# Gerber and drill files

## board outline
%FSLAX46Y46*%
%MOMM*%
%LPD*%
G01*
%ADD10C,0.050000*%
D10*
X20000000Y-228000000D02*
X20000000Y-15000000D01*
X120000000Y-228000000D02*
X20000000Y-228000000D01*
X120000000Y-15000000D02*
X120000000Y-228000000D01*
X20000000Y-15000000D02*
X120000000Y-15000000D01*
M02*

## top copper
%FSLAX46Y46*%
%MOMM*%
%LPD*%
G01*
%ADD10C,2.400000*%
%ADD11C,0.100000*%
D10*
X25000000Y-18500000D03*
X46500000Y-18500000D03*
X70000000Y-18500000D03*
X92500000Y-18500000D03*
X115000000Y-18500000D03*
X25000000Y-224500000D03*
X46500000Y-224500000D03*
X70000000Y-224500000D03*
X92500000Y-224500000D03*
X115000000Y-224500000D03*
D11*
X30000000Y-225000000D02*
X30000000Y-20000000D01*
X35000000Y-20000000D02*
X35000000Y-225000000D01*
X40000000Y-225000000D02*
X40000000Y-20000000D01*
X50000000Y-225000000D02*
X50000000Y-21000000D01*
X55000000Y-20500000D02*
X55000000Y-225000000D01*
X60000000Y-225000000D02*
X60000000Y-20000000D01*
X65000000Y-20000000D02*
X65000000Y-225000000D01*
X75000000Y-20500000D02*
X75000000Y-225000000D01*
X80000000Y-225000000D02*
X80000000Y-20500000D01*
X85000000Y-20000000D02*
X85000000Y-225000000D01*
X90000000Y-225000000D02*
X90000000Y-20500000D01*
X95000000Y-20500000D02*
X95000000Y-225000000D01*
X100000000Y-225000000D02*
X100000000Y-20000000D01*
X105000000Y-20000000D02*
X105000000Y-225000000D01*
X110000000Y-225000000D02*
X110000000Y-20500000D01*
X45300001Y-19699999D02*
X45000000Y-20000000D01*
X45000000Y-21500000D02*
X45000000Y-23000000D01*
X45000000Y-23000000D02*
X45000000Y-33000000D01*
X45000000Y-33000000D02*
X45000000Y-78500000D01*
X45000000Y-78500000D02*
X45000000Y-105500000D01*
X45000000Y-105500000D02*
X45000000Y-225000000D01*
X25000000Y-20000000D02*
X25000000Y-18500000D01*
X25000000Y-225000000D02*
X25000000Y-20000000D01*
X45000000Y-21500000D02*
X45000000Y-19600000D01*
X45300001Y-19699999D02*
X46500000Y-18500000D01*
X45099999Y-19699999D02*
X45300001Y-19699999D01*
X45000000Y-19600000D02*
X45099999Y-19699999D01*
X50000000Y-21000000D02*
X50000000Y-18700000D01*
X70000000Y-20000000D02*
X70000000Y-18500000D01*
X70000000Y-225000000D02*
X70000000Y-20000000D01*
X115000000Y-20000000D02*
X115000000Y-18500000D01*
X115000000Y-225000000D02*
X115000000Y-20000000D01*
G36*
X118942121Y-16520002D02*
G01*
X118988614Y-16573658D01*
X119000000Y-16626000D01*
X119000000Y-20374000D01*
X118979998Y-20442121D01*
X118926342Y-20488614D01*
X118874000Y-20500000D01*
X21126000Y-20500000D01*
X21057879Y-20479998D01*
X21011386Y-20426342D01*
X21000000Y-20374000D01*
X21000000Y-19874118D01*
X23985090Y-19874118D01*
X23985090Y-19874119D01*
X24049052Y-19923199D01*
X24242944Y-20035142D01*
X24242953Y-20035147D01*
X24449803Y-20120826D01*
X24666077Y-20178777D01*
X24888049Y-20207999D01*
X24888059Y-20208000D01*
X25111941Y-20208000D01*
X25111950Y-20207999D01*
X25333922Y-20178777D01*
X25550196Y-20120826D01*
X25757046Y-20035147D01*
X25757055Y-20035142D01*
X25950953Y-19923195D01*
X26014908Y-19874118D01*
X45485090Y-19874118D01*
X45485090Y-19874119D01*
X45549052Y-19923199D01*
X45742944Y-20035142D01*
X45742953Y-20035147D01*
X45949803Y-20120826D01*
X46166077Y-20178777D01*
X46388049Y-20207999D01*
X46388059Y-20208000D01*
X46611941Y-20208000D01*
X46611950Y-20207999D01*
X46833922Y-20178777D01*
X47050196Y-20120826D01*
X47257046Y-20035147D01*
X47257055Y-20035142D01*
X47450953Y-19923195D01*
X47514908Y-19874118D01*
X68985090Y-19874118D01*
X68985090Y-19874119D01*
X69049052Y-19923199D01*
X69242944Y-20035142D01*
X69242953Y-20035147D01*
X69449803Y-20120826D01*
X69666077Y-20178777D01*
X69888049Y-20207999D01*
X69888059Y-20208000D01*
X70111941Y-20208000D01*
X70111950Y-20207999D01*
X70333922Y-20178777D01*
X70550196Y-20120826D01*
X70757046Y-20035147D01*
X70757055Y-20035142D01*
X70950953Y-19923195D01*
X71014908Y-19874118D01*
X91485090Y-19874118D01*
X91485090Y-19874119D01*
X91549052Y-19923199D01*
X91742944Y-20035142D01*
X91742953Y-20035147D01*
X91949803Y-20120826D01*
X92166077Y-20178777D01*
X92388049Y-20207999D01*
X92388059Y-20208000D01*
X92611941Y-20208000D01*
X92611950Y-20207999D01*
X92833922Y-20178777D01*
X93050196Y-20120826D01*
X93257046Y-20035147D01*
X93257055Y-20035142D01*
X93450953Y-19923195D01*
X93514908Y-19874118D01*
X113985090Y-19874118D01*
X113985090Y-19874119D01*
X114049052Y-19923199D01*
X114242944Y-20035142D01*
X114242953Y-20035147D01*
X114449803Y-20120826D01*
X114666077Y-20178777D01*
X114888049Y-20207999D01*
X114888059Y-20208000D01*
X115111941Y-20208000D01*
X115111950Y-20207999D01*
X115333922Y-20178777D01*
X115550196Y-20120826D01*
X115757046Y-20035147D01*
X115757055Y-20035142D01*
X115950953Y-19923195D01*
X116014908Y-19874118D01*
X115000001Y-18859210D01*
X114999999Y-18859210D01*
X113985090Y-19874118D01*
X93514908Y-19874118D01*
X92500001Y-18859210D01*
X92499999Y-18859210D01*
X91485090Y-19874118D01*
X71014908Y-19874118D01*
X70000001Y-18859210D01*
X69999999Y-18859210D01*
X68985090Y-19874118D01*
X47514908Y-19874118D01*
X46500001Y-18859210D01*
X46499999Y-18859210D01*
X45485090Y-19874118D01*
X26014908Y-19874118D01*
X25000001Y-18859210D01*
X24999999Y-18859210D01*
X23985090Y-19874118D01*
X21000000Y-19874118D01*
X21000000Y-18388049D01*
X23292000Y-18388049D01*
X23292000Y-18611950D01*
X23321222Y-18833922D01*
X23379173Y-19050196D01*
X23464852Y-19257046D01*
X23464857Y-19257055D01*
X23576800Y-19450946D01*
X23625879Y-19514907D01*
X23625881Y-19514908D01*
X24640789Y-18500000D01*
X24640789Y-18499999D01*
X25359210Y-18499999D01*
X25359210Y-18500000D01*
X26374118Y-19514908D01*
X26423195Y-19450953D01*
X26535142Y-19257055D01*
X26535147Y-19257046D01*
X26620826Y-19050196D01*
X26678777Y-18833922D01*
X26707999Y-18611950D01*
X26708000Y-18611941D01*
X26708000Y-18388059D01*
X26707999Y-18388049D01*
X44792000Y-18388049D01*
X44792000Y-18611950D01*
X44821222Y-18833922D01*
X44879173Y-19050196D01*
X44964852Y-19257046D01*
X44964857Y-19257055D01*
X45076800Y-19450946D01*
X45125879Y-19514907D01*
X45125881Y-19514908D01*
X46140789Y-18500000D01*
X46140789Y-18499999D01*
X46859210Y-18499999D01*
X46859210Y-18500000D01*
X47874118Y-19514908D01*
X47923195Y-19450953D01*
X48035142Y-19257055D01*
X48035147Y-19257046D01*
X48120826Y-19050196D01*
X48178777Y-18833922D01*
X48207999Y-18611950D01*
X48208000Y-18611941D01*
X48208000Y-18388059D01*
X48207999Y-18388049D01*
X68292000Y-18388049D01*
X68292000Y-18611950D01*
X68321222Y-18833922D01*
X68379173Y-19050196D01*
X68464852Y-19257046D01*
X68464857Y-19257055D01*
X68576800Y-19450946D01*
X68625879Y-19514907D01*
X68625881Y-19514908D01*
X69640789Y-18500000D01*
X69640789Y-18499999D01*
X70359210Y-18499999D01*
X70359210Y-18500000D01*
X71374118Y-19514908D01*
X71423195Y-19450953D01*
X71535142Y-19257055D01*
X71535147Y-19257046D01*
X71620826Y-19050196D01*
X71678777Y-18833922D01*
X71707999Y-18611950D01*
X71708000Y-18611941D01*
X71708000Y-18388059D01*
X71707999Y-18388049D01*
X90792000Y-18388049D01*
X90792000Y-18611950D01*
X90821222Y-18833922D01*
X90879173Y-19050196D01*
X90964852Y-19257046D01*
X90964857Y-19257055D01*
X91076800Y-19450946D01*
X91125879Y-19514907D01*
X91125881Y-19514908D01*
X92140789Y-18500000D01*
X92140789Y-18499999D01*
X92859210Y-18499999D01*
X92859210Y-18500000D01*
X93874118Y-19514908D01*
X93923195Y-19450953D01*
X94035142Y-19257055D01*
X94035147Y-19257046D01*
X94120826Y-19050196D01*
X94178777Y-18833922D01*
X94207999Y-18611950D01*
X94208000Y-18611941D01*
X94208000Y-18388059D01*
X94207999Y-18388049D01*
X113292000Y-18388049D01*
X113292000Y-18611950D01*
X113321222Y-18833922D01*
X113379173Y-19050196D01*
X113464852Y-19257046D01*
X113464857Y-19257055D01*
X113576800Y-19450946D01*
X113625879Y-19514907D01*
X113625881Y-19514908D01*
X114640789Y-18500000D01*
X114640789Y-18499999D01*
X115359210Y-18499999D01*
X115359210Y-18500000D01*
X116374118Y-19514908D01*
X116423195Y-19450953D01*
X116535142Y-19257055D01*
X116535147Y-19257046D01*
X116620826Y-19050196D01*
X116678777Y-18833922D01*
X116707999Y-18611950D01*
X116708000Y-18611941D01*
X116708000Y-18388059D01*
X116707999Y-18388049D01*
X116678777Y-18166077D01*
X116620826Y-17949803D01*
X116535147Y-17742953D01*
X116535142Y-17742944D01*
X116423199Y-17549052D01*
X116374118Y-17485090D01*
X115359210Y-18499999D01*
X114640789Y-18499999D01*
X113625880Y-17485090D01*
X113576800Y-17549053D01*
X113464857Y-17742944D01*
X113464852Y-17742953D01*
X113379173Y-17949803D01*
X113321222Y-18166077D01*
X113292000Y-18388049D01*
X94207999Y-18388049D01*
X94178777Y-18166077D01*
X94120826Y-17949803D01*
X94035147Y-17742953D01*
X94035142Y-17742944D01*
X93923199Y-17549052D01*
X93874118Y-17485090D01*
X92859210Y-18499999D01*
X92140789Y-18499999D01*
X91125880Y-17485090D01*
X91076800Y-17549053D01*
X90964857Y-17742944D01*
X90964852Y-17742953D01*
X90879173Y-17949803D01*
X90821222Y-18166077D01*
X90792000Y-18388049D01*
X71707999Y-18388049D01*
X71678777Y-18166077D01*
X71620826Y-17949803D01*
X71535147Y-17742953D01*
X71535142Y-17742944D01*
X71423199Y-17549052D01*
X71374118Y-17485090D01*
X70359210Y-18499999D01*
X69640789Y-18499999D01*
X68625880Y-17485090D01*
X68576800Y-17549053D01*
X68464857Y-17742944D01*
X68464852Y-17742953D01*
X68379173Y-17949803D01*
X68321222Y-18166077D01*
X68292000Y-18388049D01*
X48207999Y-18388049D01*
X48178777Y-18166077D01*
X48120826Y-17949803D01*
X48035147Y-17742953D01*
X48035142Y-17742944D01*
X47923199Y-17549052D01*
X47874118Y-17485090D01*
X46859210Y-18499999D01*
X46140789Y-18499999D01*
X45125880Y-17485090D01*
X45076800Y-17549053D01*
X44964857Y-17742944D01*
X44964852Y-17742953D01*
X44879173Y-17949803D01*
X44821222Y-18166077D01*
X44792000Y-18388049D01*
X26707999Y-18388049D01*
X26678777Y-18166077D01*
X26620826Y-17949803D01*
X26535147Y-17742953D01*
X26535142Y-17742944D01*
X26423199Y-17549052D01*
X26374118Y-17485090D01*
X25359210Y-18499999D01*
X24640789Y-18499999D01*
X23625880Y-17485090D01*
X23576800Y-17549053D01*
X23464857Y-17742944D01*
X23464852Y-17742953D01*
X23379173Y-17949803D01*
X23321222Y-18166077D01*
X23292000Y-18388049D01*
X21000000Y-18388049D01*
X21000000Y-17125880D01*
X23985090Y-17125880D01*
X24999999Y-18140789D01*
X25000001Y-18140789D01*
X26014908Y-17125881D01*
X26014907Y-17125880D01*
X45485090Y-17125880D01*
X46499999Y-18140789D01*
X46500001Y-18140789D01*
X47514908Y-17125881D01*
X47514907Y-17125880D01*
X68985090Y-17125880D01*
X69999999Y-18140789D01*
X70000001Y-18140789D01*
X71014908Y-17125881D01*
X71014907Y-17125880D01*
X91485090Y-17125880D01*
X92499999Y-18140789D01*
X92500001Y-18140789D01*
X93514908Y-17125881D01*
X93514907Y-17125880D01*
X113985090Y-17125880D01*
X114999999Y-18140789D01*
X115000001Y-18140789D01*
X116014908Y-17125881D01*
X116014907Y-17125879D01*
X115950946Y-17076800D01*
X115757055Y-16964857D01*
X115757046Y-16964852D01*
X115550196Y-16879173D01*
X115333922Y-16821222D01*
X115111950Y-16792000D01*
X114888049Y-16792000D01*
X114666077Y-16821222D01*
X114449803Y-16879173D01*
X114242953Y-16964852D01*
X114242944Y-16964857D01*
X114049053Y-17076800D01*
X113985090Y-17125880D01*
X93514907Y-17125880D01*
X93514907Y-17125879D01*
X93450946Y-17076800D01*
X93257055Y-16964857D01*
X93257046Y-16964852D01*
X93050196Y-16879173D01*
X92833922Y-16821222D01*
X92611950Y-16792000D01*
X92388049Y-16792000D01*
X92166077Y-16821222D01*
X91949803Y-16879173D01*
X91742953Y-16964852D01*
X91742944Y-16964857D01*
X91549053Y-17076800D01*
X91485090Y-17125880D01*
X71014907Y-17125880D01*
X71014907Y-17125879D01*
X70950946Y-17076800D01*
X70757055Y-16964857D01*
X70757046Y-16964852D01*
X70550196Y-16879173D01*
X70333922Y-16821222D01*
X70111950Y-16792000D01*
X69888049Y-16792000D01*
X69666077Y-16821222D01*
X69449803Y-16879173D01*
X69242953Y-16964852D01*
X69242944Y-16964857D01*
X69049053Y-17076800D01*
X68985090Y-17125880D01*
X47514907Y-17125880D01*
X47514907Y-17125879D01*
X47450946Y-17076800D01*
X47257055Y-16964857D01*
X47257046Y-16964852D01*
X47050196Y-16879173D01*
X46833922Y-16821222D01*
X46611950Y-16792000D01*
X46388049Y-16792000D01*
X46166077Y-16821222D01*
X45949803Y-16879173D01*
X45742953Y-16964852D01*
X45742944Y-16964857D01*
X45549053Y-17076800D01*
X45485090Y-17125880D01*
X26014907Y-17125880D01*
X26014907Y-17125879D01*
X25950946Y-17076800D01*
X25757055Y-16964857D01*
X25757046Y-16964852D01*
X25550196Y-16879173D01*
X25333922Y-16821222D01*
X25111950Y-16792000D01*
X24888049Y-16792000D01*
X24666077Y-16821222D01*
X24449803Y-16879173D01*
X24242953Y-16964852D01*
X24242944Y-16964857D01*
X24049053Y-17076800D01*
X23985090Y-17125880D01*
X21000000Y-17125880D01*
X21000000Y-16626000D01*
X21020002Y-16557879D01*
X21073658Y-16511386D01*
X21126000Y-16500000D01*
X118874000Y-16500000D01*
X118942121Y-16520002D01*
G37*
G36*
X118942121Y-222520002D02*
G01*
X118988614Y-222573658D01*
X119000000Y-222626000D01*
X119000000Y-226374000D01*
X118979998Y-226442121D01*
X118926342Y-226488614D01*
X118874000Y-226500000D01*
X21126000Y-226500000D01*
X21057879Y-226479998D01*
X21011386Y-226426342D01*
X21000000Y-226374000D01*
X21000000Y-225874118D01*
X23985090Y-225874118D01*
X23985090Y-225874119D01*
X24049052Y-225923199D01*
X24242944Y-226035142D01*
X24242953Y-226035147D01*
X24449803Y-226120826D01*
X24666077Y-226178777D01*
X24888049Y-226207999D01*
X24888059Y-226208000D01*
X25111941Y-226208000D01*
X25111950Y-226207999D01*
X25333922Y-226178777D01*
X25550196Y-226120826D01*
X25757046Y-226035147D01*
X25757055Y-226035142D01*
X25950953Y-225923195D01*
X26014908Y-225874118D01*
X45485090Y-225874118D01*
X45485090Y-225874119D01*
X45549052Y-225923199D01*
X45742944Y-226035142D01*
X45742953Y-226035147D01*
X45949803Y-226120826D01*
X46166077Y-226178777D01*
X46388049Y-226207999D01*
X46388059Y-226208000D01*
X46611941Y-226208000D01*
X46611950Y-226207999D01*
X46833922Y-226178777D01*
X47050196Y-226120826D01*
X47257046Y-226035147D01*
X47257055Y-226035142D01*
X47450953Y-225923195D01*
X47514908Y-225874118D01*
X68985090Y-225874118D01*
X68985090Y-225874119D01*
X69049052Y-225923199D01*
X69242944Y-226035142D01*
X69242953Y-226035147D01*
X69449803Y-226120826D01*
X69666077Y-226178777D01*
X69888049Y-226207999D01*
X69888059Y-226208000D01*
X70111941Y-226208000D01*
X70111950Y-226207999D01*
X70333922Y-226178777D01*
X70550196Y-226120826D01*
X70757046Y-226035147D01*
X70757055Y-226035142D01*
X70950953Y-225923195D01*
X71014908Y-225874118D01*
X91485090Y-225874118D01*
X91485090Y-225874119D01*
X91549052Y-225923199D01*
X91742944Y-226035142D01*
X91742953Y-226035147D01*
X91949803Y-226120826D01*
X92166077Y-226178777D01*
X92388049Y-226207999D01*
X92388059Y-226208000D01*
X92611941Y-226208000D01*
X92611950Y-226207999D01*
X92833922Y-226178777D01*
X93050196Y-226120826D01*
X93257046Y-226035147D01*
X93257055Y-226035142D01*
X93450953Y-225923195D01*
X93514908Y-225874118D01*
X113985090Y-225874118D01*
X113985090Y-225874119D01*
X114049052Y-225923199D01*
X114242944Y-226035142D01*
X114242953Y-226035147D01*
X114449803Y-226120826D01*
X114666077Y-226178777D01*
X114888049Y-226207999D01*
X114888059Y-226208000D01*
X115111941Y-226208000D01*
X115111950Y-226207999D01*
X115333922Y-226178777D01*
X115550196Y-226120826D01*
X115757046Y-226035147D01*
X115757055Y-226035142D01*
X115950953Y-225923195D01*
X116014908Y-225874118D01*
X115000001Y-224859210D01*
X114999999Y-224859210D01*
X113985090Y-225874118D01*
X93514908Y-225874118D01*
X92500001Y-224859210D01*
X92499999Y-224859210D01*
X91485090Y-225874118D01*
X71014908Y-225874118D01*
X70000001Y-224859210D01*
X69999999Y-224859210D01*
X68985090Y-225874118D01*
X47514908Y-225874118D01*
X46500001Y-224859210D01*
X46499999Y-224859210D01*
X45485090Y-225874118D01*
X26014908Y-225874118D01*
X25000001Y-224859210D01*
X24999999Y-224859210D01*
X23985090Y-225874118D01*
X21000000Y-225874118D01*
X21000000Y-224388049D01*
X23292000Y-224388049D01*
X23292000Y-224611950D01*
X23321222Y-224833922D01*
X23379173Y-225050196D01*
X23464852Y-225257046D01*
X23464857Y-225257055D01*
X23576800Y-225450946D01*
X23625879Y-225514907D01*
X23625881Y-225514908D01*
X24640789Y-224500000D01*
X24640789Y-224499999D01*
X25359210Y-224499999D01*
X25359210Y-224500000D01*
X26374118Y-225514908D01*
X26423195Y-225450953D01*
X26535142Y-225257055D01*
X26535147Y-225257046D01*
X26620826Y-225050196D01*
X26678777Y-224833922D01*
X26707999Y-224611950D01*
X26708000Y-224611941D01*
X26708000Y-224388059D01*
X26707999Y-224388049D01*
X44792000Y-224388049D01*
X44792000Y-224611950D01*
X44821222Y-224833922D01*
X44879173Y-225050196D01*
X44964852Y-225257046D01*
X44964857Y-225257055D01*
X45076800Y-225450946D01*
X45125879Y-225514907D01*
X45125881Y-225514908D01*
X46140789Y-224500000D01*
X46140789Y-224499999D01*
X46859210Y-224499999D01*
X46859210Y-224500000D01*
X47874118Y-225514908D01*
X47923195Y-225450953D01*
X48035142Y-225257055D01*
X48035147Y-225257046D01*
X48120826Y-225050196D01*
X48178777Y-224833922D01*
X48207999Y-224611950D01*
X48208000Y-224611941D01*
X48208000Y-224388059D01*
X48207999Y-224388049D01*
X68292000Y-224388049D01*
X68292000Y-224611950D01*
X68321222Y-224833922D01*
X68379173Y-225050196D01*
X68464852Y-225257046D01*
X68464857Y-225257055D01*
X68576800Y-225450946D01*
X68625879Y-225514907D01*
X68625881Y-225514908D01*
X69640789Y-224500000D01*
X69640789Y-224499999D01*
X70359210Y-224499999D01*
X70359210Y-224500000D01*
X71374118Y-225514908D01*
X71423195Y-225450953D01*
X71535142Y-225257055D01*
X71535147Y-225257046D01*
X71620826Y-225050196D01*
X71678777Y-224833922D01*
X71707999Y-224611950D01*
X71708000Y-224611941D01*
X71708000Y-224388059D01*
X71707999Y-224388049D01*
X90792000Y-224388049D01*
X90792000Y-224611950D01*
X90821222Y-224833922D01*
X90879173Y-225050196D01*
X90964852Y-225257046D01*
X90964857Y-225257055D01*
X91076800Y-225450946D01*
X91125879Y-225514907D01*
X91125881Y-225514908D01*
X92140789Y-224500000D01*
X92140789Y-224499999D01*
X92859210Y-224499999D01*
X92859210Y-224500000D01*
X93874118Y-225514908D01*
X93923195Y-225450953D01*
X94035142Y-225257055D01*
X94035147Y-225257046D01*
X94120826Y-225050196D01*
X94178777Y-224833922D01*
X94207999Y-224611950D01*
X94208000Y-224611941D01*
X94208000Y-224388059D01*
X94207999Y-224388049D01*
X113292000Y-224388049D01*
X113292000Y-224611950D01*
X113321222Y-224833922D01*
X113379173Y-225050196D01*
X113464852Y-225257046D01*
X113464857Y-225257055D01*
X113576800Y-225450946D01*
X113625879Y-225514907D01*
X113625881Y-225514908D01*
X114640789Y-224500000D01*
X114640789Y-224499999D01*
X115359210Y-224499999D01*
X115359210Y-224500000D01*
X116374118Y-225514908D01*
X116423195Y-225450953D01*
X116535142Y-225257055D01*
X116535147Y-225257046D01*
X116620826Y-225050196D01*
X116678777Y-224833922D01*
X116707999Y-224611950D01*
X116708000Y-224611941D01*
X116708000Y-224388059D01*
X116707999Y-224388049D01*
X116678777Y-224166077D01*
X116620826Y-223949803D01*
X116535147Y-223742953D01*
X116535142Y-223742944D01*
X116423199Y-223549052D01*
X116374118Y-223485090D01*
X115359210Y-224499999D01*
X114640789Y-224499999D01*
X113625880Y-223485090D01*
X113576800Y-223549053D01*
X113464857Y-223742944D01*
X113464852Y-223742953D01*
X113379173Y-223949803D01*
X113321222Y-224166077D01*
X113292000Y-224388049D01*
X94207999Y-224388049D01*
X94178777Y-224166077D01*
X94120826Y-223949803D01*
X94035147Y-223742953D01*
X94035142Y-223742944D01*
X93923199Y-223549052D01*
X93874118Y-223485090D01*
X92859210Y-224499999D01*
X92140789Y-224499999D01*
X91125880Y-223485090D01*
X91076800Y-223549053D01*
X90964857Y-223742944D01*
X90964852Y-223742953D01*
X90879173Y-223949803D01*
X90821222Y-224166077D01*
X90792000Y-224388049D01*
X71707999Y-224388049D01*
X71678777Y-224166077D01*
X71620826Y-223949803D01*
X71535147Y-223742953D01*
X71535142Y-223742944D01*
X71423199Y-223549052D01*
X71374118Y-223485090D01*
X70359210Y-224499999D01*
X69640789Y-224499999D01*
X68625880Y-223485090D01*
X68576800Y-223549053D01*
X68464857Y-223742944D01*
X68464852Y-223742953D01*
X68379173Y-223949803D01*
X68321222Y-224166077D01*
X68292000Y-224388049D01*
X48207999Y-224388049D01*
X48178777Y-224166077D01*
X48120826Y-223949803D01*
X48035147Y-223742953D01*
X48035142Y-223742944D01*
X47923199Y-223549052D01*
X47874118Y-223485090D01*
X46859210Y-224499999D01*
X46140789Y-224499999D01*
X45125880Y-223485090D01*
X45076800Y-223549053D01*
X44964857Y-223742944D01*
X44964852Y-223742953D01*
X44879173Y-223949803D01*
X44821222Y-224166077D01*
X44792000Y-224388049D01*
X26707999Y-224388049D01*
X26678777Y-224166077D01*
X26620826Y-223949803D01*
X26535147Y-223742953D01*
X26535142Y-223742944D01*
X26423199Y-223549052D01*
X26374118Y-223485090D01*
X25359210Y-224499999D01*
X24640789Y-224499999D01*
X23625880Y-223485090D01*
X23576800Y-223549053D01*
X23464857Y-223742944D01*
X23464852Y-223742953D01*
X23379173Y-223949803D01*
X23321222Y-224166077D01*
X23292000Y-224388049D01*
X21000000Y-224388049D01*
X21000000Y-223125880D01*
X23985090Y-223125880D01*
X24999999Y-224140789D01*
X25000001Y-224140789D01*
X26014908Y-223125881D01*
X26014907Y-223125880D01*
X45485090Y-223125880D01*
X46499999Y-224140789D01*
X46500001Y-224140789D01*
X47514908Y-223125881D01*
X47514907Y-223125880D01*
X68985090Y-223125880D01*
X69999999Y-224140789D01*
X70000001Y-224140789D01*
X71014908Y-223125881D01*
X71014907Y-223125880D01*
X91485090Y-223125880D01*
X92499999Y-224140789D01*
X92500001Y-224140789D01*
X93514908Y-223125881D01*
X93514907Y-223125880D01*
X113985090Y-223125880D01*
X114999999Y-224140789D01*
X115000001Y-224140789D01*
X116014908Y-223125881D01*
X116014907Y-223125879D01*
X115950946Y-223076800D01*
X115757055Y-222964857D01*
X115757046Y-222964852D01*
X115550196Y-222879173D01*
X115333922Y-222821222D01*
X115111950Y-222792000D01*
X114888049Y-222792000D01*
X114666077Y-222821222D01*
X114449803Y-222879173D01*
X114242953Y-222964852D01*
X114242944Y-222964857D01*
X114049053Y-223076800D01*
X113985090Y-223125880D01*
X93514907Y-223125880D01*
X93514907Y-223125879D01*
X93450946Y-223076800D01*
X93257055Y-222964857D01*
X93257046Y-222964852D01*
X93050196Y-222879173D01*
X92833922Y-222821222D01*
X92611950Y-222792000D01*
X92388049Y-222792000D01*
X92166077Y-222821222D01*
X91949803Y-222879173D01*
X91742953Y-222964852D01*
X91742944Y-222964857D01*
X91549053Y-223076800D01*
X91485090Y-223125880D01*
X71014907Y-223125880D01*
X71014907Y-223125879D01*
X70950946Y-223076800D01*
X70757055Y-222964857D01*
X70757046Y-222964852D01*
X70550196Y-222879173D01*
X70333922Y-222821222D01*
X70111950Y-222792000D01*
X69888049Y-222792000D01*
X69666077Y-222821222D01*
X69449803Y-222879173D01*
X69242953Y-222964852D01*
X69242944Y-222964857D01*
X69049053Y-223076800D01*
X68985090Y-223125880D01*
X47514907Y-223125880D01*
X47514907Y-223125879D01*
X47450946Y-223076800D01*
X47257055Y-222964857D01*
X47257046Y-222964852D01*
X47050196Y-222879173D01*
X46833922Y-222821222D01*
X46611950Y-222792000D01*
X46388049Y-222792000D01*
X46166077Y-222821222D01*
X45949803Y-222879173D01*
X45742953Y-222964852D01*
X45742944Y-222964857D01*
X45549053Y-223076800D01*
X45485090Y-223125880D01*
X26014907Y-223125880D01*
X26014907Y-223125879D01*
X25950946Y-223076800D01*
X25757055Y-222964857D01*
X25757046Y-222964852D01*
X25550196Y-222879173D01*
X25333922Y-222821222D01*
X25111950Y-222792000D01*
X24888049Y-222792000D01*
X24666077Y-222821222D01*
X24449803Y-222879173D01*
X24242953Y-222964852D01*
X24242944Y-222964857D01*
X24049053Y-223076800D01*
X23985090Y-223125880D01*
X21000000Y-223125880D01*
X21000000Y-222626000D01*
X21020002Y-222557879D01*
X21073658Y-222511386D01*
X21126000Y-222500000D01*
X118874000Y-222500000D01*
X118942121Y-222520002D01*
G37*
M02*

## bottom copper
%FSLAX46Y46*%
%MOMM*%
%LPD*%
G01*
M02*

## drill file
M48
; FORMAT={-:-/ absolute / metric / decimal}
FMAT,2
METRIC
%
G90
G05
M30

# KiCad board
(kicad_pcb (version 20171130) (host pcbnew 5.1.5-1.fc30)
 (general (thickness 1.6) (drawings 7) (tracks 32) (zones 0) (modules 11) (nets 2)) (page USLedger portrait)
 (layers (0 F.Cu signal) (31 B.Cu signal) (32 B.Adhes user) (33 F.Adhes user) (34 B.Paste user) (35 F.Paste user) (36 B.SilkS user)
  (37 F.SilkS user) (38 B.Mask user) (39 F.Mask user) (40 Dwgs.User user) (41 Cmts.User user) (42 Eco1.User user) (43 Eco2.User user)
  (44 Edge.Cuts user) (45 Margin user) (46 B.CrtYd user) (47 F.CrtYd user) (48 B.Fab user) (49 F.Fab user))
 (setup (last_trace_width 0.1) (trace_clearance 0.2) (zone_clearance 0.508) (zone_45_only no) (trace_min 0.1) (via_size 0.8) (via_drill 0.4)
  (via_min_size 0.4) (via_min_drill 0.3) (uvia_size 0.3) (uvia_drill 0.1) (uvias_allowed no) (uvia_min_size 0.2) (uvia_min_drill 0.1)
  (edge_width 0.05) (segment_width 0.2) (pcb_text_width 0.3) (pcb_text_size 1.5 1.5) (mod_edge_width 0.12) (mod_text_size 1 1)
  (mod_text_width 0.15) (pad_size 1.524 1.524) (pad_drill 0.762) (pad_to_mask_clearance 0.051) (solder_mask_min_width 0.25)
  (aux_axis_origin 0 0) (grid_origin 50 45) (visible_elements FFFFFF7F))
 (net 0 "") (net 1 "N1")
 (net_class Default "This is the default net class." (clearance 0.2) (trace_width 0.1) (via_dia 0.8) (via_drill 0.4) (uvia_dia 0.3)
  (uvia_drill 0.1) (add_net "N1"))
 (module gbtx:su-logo (layer F.Cu) (at 30.5 211.5)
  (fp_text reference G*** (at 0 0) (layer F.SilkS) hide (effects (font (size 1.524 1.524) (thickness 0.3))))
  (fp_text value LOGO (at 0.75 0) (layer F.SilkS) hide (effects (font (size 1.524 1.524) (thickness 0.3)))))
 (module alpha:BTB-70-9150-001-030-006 (layer F.Cu) (at 25 18.5)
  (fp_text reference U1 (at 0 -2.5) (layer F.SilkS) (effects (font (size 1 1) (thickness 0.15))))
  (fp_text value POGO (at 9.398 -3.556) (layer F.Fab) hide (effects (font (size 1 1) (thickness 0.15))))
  (pad 1 smd circle (at 0 0) (size 2.4 2.4) (layers F.Cu F.Paste F.Mask) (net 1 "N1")))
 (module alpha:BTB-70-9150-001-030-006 (layer F.Cu) (at 46.5 18.5)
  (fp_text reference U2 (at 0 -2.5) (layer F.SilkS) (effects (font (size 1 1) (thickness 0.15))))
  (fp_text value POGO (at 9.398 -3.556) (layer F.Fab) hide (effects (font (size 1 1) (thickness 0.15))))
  (pad 1 smd circle (at 0 0) (size 2.4 2.4) (layers F.Cu F.Paste F.Mask) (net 1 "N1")))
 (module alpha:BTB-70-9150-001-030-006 (layer F.Cu) (at 70 18.5)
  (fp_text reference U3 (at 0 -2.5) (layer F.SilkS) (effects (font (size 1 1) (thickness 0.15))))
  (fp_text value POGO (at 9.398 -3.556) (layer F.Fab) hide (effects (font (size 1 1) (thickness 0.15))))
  (pad 1 smd circle (at 0 0) (size 2.4 2.4) (layers F.Cu F.Paste F.Mask) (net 1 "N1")))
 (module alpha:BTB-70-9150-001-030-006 (layer F.Cu) (at 92.5 18.5)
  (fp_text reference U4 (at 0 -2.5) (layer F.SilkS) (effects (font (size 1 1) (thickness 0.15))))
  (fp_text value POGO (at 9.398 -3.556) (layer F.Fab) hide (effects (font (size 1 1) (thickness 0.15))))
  (pad 1 smd circle (at 0 0) (size 2.4 2.4) (layers F.Cu F.Paste F.Mask) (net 1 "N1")))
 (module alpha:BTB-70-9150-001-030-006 (layer F.Cu) (at 115 18.5)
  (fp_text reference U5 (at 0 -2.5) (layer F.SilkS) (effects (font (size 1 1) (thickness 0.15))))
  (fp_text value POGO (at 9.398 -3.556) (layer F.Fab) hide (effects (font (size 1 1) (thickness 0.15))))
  (pad 1 smd circle (at 0 0) (size 2.4 2.4) (layers F.Cu F.Paste F.Mask) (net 1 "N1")))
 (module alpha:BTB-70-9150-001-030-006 (layer F.Cu) (at 25 224.5)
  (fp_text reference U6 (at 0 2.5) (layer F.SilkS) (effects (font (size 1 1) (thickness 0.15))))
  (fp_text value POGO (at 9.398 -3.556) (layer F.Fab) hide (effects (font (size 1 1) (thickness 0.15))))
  (pad 1 smd circle (at 0 0) (size 2.4 2.4) (layers F.Cu F.Paste F.Mask) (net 1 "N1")))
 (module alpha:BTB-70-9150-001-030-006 (layer F.Cu) (at 46.5 224.5)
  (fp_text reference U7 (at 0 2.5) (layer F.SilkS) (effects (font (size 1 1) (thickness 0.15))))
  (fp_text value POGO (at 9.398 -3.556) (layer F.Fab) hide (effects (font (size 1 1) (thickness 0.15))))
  (pad 1 smd circle (at 0 0) (size 2.4 2.4) (layers F.Cu F.Paste F.Mask) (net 1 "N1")))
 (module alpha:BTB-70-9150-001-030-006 (layer F.Cu) (at 70 224.5)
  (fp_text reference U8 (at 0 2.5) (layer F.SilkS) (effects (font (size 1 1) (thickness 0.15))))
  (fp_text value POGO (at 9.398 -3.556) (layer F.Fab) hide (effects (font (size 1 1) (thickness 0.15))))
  (pad 1 smd circle (at 0 0) (size 2.4 2.4) (layers F.Cu F.Paste F.Mask) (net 1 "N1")))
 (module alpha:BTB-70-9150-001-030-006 (layer F.Cu) (at 92.5 224.5)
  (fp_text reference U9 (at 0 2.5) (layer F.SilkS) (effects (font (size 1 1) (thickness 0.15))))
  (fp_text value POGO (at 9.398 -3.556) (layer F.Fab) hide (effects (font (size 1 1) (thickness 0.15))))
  (pad 1 smd circle (at 0 0) (size 2.4 2.4) (layers F.Cu F.Paste F.Mask) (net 1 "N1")))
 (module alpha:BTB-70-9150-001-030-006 (layer F.Cu) (at 115 224.5)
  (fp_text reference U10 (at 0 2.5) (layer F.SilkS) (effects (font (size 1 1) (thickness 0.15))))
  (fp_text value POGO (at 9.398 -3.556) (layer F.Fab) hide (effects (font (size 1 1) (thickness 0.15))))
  (pad 1 smd circle (at 0 0) (size 2.4 2.4) (layers F.Cu F.Paste F.Mask) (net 1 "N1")))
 (gr_line (start 20 228) (end 20 15) (layer Edge.Cuts) (width 0.05))
 (gr_line (start 120 228) (end 20 228) (layer Edge.Cuts) (width 0.05))
 (gr_line (start 120 15) (end 120 228) (layer Edge.Cuts) (width 0.05))
 (gr_line (start 20 15) (end 120 15) (layer Edge.Cuts) (width 0.05))
 (segment (start 30 225) (end 30 20) (width 0.1) (layer F.Cu) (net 1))
 (segment (start 35 20) (end 35 225) (width 0.1) (layer F.Cu) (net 1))
 (segment (start 40 225) (end 40 20) (width 0.1) (layer F.Cu) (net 1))
 (segment (start 50 225) (end 50 21) (width 0.1) (layer F.Cu) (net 1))
 (segment (start 55 20.5) (end 55 225) (width 0.1) (layer F.Cu) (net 1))
 (segment (start 60 225) (end 60 20) (width 0.1) (layer F.Cu) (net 1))
 (segment (start 65 20) (end 65 225) (width 0.1) (layer F.Cu) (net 1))
 (segment (start 75 20.5) (end 75 225) (width 0.1) (layer F.Cu) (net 1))
 (segment (start 80 225) (end 80 20.5) (width 0.1) (layer F.Cu) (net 1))
 (segment (start 85 20) (end 85 225) (width 0.1) (layer F.Cu) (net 1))
 (segment (start 90 225) (end 90 20.5) (width 0.1) (layer F.Cu) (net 1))
 (segment (start 95 20.5) (end 95 225) (width 0.1) (layer F.Cu) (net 1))
 (segment (start 100 225) (end 100 20) (width 0.1) (layer F.Cu) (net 1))
 (segment (start 105 20) (end 105 225) (width 0.1) (layer F.Cu) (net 1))
 (segment (start 110 225) (end 110 20.5) (width 0.1) (layer F.Cu) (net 1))
 (segment (start 45.300001 19.699999) (end 45 20) (width 0.1) (layer F.Cu) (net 1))
 (segment (start 45 21.5) (end 45 23) (width 0.1) (layer F.Cu) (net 1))
 (segment (start 45 23) (end 45 33) (width 0.1) (layer F.Cu) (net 1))
 (segment (start 45 33) (end 45 78.5) (width 0.1) (layer F.Cu) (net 1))
 (segment (start 45 78.5) (end 45 105.5) (width 0.1) (layer F.Cu) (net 1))
 (segment (start 45 105.5) (end 45 225) (width 0.1) (layer F.Cu) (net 1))
 (segment (start 25 20) (end 25 18.5) (width 0.1) (layer F.Cu) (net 1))
 (segment (start 25 225) (end 25 20) (width 0.1) (layer F.Cu) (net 1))
 (segment (start 45 21.5) (end 45 19.6) (width 0.1) (layer F.Cu) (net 1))
 (segment (start 45.300001 19.699999) (end 46.5 18.5) (width 0.1) (layer F.Cu) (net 1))
 (segment (start 45.099999 19.699999) (end 45.300001 19.699999) (width 0.1) (layer F.Cu) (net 1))
 (segment (start 45 19.6) (end 45.099999 19.699999) (width 0.1) (layer F.Cu) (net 1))
 (segment (start 50 21) (end 50 18.7) (width 0.1) (layer F.Cu) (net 1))
 (segment (start 70 20) (end 70 18.5) (width 0.1) (layer F.Cu) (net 1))
 (segment (start 70 225) (end 70 20) (width 0.1) (layer F.Cu) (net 1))
 (segment (start 115 20) (end 115 18.5) (width 0.1) (layer F.Cu) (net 1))
 (segment (start 115 225) (end 115 20) (width 0.1) (layer F.Cu) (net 1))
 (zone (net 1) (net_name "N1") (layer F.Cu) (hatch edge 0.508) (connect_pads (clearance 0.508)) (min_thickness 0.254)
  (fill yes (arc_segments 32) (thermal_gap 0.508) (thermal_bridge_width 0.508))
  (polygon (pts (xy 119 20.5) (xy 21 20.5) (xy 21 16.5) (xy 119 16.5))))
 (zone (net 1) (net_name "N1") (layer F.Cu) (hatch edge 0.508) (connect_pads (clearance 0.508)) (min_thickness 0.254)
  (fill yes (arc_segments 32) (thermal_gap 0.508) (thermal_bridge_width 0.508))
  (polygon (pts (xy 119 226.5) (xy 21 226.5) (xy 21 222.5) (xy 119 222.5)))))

